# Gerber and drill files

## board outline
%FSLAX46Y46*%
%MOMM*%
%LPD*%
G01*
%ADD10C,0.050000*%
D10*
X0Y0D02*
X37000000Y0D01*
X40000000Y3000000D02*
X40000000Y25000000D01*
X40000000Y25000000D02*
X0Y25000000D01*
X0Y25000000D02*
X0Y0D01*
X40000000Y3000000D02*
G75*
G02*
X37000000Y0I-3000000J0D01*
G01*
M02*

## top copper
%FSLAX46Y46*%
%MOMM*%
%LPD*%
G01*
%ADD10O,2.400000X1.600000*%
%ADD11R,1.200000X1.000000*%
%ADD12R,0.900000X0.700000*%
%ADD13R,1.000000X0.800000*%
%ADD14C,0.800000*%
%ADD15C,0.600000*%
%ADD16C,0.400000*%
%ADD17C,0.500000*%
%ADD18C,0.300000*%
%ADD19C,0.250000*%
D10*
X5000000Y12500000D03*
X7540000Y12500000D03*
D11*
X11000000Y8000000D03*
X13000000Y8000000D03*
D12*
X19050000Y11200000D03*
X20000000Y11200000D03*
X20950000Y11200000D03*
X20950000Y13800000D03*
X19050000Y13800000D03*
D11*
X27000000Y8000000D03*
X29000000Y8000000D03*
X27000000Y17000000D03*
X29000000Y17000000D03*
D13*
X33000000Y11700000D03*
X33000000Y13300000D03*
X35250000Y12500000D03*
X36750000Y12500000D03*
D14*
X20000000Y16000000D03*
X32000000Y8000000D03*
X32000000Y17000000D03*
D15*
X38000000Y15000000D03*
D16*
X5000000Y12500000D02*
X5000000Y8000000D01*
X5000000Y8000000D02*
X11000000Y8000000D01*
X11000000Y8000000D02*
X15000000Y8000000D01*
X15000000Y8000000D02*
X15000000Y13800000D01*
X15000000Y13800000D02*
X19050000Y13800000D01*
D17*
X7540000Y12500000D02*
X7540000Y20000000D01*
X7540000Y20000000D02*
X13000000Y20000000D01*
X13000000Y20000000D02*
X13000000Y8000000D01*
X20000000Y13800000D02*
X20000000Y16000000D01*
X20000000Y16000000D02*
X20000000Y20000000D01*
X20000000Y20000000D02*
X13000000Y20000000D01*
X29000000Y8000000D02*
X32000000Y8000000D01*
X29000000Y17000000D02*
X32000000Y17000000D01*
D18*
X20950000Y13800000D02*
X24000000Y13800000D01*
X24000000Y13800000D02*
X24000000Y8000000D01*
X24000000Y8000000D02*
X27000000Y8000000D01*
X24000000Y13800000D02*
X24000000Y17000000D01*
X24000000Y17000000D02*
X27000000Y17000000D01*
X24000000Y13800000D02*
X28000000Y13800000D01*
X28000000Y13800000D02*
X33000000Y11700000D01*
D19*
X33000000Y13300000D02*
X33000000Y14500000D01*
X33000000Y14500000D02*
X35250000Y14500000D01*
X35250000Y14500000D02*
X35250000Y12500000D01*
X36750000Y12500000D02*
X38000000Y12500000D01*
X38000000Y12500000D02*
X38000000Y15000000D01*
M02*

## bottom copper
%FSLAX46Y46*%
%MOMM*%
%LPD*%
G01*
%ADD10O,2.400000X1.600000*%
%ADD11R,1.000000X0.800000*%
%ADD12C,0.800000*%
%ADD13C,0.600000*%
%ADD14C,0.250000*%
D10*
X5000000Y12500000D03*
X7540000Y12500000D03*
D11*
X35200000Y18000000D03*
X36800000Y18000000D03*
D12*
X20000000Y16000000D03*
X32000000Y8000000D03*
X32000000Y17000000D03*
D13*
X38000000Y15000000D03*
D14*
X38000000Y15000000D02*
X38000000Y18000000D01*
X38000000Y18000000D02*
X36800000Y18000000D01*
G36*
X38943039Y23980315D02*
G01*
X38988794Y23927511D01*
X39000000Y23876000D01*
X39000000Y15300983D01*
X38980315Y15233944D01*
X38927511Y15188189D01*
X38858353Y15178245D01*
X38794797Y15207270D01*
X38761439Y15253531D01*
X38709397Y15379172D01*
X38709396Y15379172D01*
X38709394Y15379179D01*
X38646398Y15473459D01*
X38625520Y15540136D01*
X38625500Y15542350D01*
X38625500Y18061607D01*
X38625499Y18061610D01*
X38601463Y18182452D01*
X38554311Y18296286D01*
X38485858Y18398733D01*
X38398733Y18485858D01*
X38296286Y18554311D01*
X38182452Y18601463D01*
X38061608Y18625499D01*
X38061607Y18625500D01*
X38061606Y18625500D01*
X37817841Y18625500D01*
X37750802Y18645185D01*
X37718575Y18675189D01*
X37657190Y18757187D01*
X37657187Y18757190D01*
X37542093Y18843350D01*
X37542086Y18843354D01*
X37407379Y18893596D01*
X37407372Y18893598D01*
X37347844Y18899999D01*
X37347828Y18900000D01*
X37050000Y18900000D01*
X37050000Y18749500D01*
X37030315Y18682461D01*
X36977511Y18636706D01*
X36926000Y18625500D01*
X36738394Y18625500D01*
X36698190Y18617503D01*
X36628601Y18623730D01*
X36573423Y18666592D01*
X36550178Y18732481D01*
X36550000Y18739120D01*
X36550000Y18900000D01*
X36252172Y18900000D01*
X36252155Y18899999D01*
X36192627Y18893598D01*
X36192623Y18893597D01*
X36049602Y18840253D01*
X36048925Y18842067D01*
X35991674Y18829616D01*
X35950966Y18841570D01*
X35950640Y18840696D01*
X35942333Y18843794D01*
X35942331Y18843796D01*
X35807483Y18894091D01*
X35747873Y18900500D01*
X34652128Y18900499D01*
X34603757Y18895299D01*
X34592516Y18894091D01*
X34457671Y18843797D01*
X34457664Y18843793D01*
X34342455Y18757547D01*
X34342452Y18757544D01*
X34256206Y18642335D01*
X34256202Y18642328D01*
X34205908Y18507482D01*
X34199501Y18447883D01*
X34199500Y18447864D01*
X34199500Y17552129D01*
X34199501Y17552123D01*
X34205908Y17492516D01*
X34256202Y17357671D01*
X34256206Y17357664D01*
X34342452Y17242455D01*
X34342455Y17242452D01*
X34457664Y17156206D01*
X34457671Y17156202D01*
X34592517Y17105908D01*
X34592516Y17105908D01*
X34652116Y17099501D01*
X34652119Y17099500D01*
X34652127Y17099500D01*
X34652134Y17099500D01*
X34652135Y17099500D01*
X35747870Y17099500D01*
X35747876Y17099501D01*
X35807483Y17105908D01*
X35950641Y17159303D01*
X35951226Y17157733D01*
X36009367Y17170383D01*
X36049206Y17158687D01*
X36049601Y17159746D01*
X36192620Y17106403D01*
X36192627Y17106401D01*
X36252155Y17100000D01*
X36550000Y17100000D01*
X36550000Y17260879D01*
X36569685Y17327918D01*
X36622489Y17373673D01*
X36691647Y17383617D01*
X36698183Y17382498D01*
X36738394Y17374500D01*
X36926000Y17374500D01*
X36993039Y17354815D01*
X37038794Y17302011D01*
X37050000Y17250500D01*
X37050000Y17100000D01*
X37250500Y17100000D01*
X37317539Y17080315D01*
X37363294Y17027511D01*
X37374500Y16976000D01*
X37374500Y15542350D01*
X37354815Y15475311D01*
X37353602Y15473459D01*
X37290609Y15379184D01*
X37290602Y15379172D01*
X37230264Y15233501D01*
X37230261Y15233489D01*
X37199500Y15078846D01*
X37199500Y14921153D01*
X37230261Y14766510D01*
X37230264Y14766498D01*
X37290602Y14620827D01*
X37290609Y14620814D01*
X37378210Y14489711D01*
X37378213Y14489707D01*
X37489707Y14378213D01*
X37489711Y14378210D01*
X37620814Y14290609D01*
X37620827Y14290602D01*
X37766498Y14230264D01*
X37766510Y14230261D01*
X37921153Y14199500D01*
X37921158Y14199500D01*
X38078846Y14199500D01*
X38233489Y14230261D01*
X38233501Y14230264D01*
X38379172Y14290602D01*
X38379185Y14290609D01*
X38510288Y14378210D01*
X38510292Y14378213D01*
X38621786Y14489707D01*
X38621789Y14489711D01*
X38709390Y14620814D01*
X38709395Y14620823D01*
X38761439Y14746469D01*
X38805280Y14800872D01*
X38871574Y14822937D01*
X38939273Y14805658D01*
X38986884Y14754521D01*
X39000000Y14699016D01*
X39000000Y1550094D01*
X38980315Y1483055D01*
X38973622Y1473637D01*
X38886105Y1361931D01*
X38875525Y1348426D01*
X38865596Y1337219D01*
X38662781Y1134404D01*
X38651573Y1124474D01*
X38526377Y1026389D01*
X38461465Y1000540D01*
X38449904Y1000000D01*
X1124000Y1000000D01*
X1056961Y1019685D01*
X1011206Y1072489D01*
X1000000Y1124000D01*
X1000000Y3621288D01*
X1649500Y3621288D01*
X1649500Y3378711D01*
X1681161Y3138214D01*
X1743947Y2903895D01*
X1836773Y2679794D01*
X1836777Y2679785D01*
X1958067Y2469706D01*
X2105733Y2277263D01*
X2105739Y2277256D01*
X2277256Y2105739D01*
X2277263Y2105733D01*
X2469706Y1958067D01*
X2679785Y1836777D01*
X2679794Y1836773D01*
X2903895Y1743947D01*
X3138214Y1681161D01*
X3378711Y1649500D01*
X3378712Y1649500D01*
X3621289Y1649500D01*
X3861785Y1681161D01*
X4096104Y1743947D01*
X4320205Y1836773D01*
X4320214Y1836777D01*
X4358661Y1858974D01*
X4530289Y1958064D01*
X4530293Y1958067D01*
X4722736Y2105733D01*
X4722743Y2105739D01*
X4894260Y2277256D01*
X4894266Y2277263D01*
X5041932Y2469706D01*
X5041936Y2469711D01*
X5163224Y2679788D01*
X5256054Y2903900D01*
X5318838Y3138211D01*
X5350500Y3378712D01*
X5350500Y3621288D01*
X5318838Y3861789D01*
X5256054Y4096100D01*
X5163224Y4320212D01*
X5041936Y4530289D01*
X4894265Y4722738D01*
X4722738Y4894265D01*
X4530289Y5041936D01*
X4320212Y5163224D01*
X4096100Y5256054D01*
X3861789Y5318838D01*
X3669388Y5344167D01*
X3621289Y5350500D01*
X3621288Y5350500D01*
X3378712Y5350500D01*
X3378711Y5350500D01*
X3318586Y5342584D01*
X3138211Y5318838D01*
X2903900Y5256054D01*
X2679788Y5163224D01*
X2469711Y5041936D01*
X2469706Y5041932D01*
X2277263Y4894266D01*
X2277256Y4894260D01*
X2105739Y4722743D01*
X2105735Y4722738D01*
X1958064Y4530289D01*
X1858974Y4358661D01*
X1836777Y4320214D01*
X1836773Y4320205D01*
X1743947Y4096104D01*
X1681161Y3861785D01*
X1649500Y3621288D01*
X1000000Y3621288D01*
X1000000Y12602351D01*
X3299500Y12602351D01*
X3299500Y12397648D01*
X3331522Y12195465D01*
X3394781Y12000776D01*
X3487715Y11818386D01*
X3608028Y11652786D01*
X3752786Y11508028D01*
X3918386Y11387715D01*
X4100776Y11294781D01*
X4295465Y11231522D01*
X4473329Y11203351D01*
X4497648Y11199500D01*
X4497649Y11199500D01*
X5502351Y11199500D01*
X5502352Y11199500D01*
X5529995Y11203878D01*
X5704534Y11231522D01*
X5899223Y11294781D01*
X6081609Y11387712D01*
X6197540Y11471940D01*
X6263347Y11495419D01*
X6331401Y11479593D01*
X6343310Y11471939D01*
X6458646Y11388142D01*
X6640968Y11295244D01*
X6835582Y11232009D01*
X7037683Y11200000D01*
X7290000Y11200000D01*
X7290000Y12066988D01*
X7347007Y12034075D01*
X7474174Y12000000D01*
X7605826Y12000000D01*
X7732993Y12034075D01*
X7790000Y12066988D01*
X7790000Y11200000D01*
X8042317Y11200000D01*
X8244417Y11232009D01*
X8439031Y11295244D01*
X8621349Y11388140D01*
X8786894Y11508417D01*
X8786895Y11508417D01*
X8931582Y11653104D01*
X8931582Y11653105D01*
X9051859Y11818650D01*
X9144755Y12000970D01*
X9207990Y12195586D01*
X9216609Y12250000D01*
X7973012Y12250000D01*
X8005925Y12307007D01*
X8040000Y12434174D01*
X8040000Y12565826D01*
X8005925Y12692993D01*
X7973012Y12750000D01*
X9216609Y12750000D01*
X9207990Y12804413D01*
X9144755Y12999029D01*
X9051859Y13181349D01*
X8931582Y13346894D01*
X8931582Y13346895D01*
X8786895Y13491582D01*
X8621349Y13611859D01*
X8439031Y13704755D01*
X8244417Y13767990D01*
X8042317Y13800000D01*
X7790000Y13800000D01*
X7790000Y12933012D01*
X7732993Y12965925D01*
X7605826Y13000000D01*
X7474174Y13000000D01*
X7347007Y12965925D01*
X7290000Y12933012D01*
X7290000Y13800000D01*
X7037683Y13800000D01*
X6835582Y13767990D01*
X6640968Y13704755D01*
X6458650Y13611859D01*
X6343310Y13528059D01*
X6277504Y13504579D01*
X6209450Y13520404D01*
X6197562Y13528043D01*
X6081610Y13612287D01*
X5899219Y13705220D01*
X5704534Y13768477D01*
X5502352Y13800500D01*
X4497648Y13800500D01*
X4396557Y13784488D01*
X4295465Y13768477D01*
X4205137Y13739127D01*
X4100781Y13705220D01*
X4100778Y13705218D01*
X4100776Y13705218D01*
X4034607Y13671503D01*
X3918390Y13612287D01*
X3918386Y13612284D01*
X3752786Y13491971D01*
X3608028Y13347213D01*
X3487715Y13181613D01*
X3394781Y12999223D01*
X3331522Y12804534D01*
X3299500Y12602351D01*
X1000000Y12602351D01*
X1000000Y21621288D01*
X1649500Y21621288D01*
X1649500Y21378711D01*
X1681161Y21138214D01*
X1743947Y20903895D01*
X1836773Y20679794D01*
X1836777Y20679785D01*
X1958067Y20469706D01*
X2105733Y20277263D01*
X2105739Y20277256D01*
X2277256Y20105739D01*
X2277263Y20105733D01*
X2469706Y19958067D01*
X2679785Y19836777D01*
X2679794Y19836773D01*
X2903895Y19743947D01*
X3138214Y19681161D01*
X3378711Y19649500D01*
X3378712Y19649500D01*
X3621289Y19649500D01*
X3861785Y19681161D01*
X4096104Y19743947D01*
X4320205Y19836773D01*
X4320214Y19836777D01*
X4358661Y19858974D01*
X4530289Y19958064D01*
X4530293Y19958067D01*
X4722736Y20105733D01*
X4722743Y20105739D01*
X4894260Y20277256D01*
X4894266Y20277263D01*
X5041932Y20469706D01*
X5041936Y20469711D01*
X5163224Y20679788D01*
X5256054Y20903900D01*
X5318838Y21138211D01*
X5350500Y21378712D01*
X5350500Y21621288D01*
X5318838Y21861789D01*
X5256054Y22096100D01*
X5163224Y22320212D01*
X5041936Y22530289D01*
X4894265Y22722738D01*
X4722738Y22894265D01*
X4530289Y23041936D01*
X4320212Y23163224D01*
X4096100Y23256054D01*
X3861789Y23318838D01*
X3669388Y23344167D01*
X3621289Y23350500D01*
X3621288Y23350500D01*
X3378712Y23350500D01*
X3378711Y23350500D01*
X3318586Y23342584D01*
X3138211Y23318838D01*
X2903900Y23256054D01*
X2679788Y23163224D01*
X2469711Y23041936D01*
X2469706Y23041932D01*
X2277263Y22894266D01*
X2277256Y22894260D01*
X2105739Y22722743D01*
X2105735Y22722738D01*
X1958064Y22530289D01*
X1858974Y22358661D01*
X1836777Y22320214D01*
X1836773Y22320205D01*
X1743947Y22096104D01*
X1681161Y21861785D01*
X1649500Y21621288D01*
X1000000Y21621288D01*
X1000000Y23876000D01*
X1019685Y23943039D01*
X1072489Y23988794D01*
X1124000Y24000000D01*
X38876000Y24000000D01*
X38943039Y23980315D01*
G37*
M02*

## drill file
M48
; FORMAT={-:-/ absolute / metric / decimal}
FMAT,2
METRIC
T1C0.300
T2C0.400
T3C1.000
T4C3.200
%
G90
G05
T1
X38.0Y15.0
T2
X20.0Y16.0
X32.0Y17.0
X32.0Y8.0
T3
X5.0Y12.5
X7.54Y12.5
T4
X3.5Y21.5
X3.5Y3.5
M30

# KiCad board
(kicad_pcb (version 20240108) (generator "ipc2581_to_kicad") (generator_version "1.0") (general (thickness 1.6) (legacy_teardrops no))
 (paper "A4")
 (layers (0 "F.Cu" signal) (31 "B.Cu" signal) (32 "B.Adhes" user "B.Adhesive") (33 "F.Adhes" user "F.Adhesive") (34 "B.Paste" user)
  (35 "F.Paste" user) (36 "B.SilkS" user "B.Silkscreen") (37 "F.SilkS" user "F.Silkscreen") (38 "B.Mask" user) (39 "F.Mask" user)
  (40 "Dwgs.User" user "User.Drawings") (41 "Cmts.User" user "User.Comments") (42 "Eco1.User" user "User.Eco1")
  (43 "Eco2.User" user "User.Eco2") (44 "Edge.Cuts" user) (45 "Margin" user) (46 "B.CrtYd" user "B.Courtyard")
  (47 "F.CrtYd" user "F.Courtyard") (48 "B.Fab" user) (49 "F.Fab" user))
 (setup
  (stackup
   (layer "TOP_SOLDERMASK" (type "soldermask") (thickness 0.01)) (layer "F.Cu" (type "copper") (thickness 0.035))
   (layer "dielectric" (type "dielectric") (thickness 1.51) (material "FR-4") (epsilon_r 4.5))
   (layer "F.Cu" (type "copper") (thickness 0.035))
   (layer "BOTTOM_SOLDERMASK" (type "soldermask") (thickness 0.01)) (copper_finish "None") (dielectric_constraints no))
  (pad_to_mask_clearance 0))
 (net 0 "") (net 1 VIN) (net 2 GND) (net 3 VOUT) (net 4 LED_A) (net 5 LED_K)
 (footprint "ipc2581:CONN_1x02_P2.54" (layer "F.Cu") (at 5 -12.5)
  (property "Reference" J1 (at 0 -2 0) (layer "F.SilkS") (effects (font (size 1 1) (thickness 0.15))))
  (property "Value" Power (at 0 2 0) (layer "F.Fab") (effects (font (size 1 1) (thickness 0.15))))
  (pad 1 thru_hole oval (at 0 0) (size 2.4 1.6) (drill 1) (layers "*.Cu" "*.Mask") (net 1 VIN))
  (pad 2 thru_hole oval (at 2.54 0) (size 2.4 1.6) (drill 1) (layers "*.Cu" "*.Mask") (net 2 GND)))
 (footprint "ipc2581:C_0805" (layer "F.Cu") (at 12 -8)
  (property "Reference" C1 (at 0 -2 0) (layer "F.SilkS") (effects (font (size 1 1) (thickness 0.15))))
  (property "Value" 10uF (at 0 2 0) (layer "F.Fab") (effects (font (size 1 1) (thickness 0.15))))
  (pad 1 smd rect (at -1 0) (size 1.2 1) (layers "F.Cu" "F.Paste" "F.Mask") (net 1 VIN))
  (pad 2 smd rect (at 1 0) (size 1.2 1) (layers "F.Cu" "F.Paste" "F.Mask") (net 2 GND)))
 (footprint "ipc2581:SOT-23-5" (layer "F.Cu") (at 20 -12.5)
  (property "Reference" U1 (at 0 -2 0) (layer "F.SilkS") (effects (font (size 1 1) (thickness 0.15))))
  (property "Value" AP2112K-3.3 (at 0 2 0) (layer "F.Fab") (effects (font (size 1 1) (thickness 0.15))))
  (pad 1 smd rect (at -0.95 1.3) (size 0.9 0.7) (layers "F.Cu" "F.Paste" "F.Mask") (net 1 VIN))
  (pad 2 smd rect (at 0 1.3) (size 0.9 0.7) (layers "F.Cu" "F.Paste" "F.Mask") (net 2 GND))
  (pad 3 smd rect (at 0.95 1.3) (size 0.9 0.7) (layers "F.Cu" "F.Paste" "F.Mask") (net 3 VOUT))
  (pad 4 smd rect (at 0.95 -1.3) (size 0.9 0.7) (layers "F.Cu" "F.Paste" "F.Mask"))
  (pad 5 smd rect (at -0.95 -1.3) (size 0.9 0.7) (layers "F.Cu" "F.Paste" "F.Mask")))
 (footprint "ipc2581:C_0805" (layer "F.Cu") (at 28 -8)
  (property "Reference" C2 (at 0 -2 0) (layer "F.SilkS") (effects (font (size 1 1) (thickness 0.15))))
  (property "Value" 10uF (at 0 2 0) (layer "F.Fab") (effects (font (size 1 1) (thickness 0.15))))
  (pad 1 smd rect (at -1 0) (size 1.2 1) (layers "F.Cu" "F.Paste" "F.Mask") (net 3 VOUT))
  (pad 2 smd rect (at 1 0) (size 1.2 1) (layers "F.Cu" "F.Paste" "F.Mask") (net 2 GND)))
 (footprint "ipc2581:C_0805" (layer "F.Cu") (at 28 -17)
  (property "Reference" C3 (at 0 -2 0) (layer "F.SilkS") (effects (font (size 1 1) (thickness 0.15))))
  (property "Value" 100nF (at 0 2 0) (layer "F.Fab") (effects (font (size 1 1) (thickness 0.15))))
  (pad 1 smd rect (at -1 0) (size 1.2 1) (layers "F.Cu" "F.Paste" "F.Mask") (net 3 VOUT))
  (pad 2 smd rect (at 1 0) (size 1.2 1) (layers "F.Cu" "F.Paste" "F.Mask") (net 2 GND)))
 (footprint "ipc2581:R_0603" (layer "F.Cu") (at 33 -12.5 90)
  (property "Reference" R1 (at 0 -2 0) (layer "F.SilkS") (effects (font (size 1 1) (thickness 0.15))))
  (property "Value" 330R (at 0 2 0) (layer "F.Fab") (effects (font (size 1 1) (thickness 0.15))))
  (pad 1 smd rect (at -0.8 0) (size 1 0.8) (layers "F.Cu" "F.Paste" "F.Mask") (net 3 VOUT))
  (pad 2 smd rect (at 0.8 0) (size 1 0.8) (layers "F.Cu" "F.Paste" "F.Mask") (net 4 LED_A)))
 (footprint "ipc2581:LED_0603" (layer "F.Cu") (at 36 -12.5)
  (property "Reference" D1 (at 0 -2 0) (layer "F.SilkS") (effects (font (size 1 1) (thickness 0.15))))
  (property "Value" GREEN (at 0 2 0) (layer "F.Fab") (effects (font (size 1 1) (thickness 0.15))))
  (pad 1 smd rect (at -0.75 0) (size 1 0.8) (layers "F.Cu" "F.Paste" "F.Mask") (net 4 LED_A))
  (pad 2 smd rect (at 0.75 0) (size 1 0.8) (layers "F.Cu" "F.Paste" "F.Mask") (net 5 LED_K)))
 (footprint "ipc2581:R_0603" (layer "B.Cu") (at 36 -18)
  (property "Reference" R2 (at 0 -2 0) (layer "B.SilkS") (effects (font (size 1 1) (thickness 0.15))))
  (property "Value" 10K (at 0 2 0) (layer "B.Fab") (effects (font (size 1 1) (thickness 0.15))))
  (pad 1 smd rect (at -0.8 0) (size 1 0.8) (layers "B.Cu" "B.Paste" "B.Mask") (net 5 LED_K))
  (pad 2 smd rect (at 0.8 0) (size 1 0.8) (layers "B.Cu" "B.Paste" "B.Mask") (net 2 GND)))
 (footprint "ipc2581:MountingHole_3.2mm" (layer "F.Cu") (at 3.5 -3.5)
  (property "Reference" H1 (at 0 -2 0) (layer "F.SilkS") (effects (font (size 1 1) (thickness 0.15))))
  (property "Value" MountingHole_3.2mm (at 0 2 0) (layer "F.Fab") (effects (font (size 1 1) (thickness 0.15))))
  (pad 1 np_thru_hole circle (at 0 0) (size 3.2 3.2) (drill 3.2) (layers "*.Cu" "*.Mask")))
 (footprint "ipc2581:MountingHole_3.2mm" (layer "F.Cu") (at 3.5 -21.5)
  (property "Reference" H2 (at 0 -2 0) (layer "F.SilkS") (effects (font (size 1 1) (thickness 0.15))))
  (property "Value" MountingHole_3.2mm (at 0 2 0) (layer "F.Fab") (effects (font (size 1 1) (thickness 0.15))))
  (pad 1 np_thru_hole circle (at 0 0) (size 3.2 3.2) (drill 3.2) (layers "*.Cu" "*.Mask")))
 (gr_line (start 0 0) (end 37 0) (stroke (width 0.05) (type solid)) (layer "Edge.Cuts"))
 (gr_line (start 40 -3) (end 40 -25) (stroke (width 0.05) (type solid)) (layer "Edge.Cuts"))
 (gr_line (start 40 -25) (end 0 -25) (stroke (width 0.05) (type solid)) (layer "Edge.Cuts"))
 (gr_line (start 0 -25) (end 0 0) (stroke (width 0.05) (type solid)) (layer "Edge.Cuts"))
 (gr_arc (start 37 0) (mid 39.12132 -0.87868) (end 40 -3) (stroke (width 0.05) (type solid)) (layer "Edge.Cuts"))
 (segment (start 5 -12.5) (end 5 -8) (width 0.4) (layer "F.Cu") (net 1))
 (segment (start 5 -8) (end 11 -8) (width 0.4) (layer "F.Cu") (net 1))
 (segment (start 11 -8) (end 15 -8) (width 0.4) (layer "F.Cu") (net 1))
 (segment (start 15 -8) (end 15 -13.8) (width 0.4) (layer "F.Cu") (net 1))
 (segment (start 15 -13.8) (end 19.05 -13.8) (width 0.4) (layer "F.Cu") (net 1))
 (segment (start 7.54 -12.5) (end 7.54 -20) (width 0.5) (layer "F.Cu") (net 2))
 (segment (start 7.54 -20) (end 13 -20) (width 0.5) (layer "F.Cu") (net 2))
 (segment (start 13 -20) (end 13 -8) (width 0.5) (layer "F.Cu") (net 2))
 (segment (start 20 -13.8) (end 20 -16) (width 0.5) (layer "F.Cu") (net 2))
 (segment (start 20 -16) (end 20 -20) (width 0.5) (layer "F.Cu") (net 2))
 (segment (start 20 -20) (end 13 -20) (width 0.5) (layer "F.Cu") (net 2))
 (segment (start 29 -8) (end 32 -8) (width 0.5) (layer "F.Cu") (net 2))
 (segment (start 29 -17) (end 32 -17) (width 0.5) (layer "F.Cu") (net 2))
 (segment (start 20.95 -13.8) (end 24 -13.8) (width 0.3) (layer "F.Cu") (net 3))
 (segment (start 24 -13.8) (end 24 -8) (width 0.3) (layer "F.Cu") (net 3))
 (segment (start 24 -8) (end 27 -8) (width 0.3) (layer "F.Cu") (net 3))
 (segment (start 24 -13.8) (end 24 -17) (width 0.3) (layer "F.Cu") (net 3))
 (segment (start 24 -17) (end 27 -17) (width 0.3) (layer "F.Cu") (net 3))
 (segment (start 24 -13.8) (end 28 -13.8) (width 0.3) (layer "F.Cu") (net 3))
 (segment (start 28 -13.8) (end 33 -11.7) (width 0.3) (layer "F.Cu") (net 3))
 (segment (start 33 -13.3) (end 33 -14.5) (width 0.25) (layer "F.Cu") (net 4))
 (segment (start 33 -14.5) (end 35.25 -14.5) (width 0.25) (layer "F.Cu") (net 4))
 (segment (start 35.25 -14.5) (end 35.25 -12.5) (width 0.25) (layer "F.Cu") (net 4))
 (segment (start 36.75 -12.5) (end 38 -12.5) (width 0.25) (layer "F.Cu") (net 5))
 (segment (start 38 -12.5) (end 38 -15) (width 0.25) (layer "F.Cu") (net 5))
 (segment (start 38 -15) (end 38 -18) (width 0.25) (layer "B.Cu") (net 5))
 (segment (start 38 -18) (end 36.8 -18) (width 0.25) (layer "B.Cu") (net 5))
 (via (at 20 -16) (size 0.8) (drill 0.4) (layers "F.Cu" "B.Cu") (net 2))
 (via (at 32 -8) (size 0.8) (drill 0.4) (layers "F.Cu" "B.Cu") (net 2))
 (via (at 32 -17) (size 0.8) (drill 0.4) (layers "F.Cu" "B.Cu") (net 2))
 (via (at 38 -15) (size 0.6) (drill 0.3) (layers "F.Cu" "B.Cu") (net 5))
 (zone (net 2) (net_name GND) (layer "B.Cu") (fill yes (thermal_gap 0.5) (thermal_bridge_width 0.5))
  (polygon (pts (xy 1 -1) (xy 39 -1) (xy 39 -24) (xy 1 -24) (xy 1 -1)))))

